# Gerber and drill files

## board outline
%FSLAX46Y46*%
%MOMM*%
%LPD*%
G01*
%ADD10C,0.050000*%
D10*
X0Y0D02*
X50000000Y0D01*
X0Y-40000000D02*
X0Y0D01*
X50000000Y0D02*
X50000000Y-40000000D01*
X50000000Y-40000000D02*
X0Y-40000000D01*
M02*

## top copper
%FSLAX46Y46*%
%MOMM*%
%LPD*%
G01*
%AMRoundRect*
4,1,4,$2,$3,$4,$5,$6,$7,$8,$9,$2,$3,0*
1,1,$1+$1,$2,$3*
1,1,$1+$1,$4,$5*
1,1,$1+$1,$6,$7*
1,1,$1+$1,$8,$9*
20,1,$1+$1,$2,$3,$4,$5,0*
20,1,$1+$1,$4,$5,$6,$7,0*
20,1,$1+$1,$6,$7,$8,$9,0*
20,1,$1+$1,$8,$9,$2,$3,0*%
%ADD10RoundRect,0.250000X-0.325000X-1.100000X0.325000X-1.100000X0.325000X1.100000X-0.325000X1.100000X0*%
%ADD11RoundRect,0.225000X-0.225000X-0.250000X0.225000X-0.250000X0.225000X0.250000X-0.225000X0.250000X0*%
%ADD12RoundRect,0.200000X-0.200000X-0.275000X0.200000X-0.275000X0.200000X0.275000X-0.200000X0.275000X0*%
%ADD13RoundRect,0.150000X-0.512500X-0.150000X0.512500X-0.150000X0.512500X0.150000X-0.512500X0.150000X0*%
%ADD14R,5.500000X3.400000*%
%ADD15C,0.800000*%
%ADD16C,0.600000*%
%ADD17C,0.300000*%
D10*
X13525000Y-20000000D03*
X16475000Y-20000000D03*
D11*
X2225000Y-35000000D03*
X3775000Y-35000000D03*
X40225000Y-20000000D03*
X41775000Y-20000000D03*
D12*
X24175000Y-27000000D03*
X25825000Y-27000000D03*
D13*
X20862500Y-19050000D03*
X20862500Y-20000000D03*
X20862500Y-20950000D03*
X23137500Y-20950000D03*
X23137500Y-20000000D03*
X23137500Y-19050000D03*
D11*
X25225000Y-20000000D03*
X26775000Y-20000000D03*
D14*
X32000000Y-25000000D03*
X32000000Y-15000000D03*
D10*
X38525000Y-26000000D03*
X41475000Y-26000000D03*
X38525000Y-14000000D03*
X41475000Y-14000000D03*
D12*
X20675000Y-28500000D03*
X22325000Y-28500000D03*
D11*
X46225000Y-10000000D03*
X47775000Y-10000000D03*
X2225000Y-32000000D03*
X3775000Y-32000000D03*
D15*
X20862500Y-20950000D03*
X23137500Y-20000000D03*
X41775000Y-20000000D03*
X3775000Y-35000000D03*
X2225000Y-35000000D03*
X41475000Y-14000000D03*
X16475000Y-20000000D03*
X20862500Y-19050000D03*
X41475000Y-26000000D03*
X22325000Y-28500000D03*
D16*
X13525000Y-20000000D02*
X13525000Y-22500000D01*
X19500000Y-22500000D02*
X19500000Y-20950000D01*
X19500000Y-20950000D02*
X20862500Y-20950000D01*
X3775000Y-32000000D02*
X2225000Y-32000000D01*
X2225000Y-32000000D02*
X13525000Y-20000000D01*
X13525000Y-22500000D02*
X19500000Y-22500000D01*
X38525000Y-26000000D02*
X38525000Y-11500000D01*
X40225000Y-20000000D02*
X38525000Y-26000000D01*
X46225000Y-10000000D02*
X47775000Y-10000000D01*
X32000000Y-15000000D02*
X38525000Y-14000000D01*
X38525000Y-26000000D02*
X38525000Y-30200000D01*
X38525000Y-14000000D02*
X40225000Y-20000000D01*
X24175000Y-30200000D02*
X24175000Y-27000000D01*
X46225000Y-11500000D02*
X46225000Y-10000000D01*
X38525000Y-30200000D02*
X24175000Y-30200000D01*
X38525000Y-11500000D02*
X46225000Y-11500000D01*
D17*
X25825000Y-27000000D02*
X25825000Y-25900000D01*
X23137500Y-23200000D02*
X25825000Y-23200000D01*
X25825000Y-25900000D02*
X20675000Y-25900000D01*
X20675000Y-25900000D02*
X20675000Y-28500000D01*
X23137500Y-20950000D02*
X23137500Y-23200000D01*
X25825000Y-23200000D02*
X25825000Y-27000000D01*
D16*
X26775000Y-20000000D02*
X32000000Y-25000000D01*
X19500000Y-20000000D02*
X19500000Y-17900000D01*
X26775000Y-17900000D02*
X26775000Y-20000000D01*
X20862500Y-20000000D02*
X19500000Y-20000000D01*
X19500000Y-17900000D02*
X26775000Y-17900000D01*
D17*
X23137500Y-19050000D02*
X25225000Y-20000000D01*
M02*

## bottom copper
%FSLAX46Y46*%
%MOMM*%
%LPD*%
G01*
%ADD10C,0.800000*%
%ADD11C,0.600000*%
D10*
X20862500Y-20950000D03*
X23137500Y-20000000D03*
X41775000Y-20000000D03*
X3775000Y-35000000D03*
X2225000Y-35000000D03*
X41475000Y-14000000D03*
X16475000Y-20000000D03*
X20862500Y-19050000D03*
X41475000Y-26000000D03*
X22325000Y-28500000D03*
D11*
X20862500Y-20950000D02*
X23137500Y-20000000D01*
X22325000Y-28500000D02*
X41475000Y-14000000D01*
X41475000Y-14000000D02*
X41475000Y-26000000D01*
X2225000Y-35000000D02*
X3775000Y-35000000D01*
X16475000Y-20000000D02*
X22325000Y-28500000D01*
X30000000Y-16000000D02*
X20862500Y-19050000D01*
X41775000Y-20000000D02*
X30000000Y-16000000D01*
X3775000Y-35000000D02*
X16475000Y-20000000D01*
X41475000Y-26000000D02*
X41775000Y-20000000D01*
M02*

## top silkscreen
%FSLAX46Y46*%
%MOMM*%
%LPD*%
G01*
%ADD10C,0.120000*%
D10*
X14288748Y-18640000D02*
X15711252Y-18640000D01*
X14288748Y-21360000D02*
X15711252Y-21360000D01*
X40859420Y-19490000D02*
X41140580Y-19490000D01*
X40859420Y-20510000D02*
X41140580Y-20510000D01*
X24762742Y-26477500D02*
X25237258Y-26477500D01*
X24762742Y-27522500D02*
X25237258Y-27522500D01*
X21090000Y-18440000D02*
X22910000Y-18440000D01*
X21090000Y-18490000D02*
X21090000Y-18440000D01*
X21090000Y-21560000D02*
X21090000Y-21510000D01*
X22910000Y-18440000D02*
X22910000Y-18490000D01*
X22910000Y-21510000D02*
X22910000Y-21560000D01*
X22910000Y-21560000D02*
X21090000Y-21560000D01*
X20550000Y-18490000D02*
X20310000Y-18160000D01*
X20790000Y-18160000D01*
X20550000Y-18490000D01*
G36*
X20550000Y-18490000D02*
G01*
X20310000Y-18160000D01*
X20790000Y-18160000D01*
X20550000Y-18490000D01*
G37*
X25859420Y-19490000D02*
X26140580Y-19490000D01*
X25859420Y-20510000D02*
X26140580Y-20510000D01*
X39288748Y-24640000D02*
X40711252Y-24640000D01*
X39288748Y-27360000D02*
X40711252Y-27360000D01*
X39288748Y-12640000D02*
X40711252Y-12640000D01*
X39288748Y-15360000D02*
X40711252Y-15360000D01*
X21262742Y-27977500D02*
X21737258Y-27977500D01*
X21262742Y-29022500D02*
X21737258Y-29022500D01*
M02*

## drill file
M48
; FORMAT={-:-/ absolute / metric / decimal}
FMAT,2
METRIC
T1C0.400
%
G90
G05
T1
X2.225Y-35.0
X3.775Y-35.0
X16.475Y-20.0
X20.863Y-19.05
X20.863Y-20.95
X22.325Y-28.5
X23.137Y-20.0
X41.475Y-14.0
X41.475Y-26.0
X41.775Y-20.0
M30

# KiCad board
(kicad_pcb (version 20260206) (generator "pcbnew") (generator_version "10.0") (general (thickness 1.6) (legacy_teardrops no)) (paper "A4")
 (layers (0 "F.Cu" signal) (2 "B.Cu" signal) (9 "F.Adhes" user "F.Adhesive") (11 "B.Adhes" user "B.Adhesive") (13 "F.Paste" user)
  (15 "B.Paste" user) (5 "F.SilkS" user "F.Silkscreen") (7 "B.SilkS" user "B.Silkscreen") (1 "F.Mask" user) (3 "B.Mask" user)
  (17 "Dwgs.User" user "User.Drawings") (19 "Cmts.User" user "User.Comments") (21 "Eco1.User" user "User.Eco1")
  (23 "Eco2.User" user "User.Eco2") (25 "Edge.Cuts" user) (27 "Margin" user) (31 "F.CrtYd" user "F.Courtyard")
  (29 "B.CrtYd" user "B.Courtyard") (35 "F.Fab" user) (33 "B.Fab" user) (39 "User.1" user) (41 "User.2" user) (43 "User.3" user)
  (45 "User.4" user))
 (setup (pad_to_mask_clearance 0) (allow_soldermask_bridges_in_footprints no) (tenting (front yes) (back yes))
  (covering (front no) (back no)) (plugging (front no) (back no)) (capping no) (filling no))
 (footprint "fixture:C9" (layer "F.Cu") (at 15 20)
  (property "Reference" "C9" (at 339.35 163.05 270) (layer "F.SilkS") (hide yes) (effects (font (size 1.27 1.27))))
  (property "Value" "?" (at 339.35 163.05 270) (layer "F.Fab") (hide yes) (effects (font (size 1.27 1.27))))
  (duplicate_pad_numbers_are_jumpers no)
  (fp_line (start -0.711252 -1.36) (end 0.711252 -1.36) (stroke (width 0.12) (type solid)) (layer "F.SilkS"))
  (fp_line (start -0.711252 1.36) (end 0.711252 1.36) (stroke (width 0.12) (type solid)) (layer "F.SilkS"))
  (pad "1" smd roundrect (at -1.475 0) (size 1.15 2.7) (layers "F.Cu" "F.Mask" "F.Paste") (roundrect_rratio 0.217391) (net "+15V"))
  (pad "2" smd roundrect (at 1.475 0) (size 1.15 2.7) (layers "F.Cu" "F.Mask" "F.Paste") (roundrect_rratio 0.217391) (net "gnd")))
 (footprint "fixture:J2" (layer "F.Cu") (at 3 35)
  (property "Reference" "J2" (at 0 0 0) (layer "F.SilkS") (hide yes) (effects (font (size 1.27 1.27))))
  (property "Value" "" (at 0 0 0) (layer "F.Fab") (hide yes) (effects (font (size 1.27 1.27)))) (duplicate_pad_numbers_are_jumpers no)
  (pad "1" smd roundrect (at -0.775 0) (size 0.9 0.95) (layers "F.Cu" "F.Mask" "F.Paste") (roundrect_rratio 0.25) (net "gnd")
   (thermal_bridge_angle 45))
  (pad "2" smd roundrect (at 0.775 0) (size 0.9 0.95) (layers "F.Cu" "F.Mask" "F.Paste") (roundrect_rratio 0.25) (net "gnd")
   (thermal_bridge_angle 45)))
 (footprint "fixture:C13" (layer "F.Cu") (at 41 20)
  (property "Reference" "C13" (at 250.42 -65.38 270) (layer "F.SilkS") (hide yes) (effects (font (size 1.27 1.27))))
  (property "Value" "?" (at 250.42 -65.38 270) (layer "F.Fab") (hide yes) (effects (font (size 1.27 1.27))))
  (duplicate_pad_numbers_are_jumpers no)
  (fp_line (start -0.14058 -0.51) (end 0.14058 -0.51) (stroke (width 0.12) (type solid)) (layer "F.SilkS"))
  (fp_line (start -0.14058 0.51) (end 0.14058 0.51) (stroke (width 0.12) (type solid)) (layer "F.SilkS"))
  (pad "1" smd roundrect (at -0.775 0) (size 0.9 0.95) (layers "F.Cu" "F.Mask" "F.Paste") (roundrect_rratio 0.25) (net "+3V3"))
  (pad "2" smd roundrect (at 0.775 0) (size 0.9 0.95) (layers "F.Cu" "F.Mask" "F.Paste") (roundrect_rratio 0.25) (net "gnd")))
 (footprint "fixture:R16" (layer "F.Cu") (at 25 27)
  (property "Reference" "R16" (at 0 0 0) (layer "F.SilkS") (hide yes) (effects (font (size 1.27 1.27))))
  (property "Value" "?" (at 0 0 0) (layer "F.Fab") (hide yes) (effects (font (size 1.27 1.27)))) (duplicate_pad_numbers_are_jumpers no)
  (fp_line (start -0.237258 -0.5225) (end 0.237258 -0.5225) (stroke (width 0.12) (type solid)) (layer "F.SilkS"))
  (fp_line (start -0.237258 0.5225) (end 0.237258 0.5225) (stroke (width 0.12) (type solid)) (layer "F.SilkS"))
  (pad "1" smd roundrect (at -0.825 0) (size 0.8 0.95) (layers "F.Cu" "F.Mask" "F.Paste") (roundrect_rratio 0.25) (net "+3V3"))
  (pad "2" smd roundrect (at 0.825 0) (size 0.8 0.95) (layers "F.Cu" "F.Mask" "F.Paste") (roundrect_rratio 0.25) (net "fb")))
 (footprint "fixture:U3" (layer "F.Cu") (at 22 20)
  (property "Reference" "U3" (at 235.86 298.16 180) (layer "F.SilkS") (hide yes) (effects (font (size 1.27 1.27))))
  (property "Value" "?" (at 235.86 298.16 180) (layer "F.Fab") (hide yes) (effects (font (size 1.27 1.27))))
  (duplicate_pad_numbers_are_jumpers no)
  (fp_line (start -0.91 -1.56) (end 0.91 -1.56) (stroke (width 0.12) (type solid)) (layer "F.SilkS"))
  (fp_line (start -0.91 -1.51) (end -0.91 -1.56) (stroke (width 0.12) (type solid)) (layer "F.SilkS"))
  (fp_line (start -0.91 1.56) (end -0.91 1.51) (stroke (width 0.12) (type solid)) (layer "F.SilkS"))
  (fp_line (start 0.91 -1.56) (end 0.91 -1.51) (stroke (width 0.12) (type solid)) (layer "F.SilkS"))
  (fp_line (start 0.91 1.51) (end 0.91 1.56) (stroke (width 0.12) (type solid)) (layer "F.SilkS"))
  (fp_line (start 0.91 1.56) (end -0.91 1.56) (stroke (width 0.12) (type solid)) (layer "F.SilkS"))
  (fp_poly (pts (xy -1.45 -1.51) (xy -1.69 -1.84) (xy -1.21 -1.84)) (stroke (width 0.12) (type solid)) (fill yes) (layer "F.SilkS"))
  (pad "1" smd roundrect (at -1.1375 -0.95) (size 1.325 0.6) (layers "F.Cu" "F.Mask" "F.Paste") (roundrect_rratio 0.25) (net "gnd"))
  (pad "2" smd roundrect (at -1.1375 0) (size 1.325 0.6) (layers "F.Cu" "F.Mask" "F.Paste") (roundrect_rratio 0.25) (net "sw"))
  (pad "3" smd roundrect (at -1.1375 0.95) (size 1.325 0.6) (layers "F.Cu" "F.Mask" "F.Paste") (roundrect_rratio 0.25) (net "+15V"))
  (pad "4" smd roundrect (at 1.1375 0.95) (size 1.325 0.6) (layers "F.Cu" "F.Mask" "F.Paste") (roundrect_rratio 0.25) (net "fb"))
  (pad "5" smd roundrect (at 1.1375 0) (size 1.325 0.6) (layers "F.Cu" "F.Mask" "F.Paste") (roundrect_rratio 0.25) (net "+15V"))
  (pad "6" smd roundrect (at 1.1375 -0.95) (size 1.325 0.6) (layers "F.Cu" "F.Mask" "F.Paste") (roundrect_rratio 0.25) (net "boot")))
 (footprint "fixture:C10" (layer "F.Cu") (at 26 20)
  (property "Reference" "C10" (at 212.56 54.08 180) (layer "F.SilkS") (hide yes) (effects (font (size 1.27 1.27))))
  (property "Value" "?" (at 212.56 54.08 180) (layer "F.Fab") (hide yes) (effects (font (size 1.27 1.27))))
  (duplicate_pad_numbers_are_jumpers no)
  (fp_line (start -0.14058 -0.51) (end 0.14058 -0.51) (stroke (width 0.12) (type solid)) (layer "F.SilkS"))
  (fp_line (start -0.14058 0.51) (end 0.14058 0.51) (stroke (width 0.12) (type solid)) (layer "F.SilkS"))
  (pad "1" smd roundrect (at -0.775 0) (size 0.9 0.95) (layers "F.Cu" "F.Mask" "F.Paste") (roundrect_rratio 0.25) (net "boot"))
  (pad "2" smd roundrect (at 0.775 0) (size 0.9 0.95) (layers "F.Cu" "F.Mask" "F.Paste") (roundrect_rratio 0.25) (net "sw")))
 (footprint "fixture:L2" (layer "F.Cu") (at 32 20 90)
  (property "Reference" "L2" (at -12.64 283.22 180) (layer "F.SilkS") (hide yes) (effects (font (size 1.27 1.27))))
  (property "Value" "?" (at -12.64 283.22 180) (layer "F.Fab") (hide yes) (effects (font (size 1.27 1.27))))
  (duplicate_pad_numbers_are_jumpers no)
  (pad "1" smd rect (at -5 0 90) (size 3.4 5.5) (layers "F.Cu" "F.Mask" "F.Paste") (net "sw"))
  (pad "2" smd rect (at 5 0 90) (size 3.4 5.5) (layers "F.Cu" "F.Mask" "F.Paste") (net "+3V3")))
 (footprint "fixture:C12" (layer "F.Cu") (at 40 26)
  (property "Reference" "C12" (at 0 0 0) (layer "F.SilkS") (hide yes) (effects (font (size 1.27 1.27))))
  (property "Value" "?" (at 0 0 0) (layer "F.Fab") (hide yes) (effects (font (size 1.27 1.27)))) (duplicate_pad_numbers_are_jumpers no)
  (fp_line (start -0.711252 -1.36) (end 0.711252 -1.36) (stroke (width 0.12) (type solid)) (layer "F.SilkS"))
  (fp_line (start -0.711252 1.36) (end 0.711252 1.36) (stroke (width 0.12) (type solid)) (layer "F.SilkS"))
  (pad "1" smd roundrect (at -1.475 0) (size 1.15 2.7) (layers "F.Cu" "F.Mask" "F.Paste") (roundrect_rratio 0.217391) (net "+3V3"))
  (pad "2" smd roundrect (at 1.475 0) (size 1.15 2.7) (layers "F.Cu" "F.Mask" "F.Paste") (roundrect_rratio 0.217391) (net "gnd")))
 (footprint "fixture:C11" (layer "F.Cu") (at 40 14)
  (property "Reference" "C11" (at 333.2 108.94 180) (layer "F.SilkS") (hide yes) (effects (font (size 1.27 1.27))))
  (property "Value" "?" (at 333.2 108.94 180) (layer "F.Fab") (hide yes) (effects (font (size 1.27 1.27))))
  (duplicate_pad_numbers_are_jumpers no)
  (fp_line (start -0.711252 -1.36) (end 0.711252 -1.36) (stroke (width 0.12) (type solid)) (layer "F.SilkS"))
  (fp_line (start -0.711252 1.36) (end 0.711252 1.36) (stroke (width 0.12) (type solid)) (layer "F.SilkS"))
  (pad "1" smd roundrect (at -1.475 0) (size 1.15 2.7) (layers "F.Cu" "F.Mask" "F.Paste") (roundrect_rratio 0.217391) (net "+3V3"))
  (pad "2" smd roundrect (at 1.475 0) (size 1.15 2.7) (layers "F.Cu" "F.Mask" "F.Paste") (roundrect_rratio 0.217391) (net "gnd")))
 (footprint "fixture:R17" (layer "F.Cu") (at 21.5 28.5)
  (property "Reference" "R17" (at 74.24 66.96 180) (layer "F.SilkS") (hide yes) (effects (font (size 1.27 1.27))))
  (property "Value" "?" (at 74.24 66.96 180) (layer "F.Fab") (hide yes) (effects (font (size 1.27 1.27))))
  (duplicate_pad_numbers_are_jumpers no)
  (fp_line (start -0.237258 -0.5225) (end 0.237258 -0.5225) (stroke (width 0.12) (type solid)) (layer "F.SilkS"))
  (fp_line (start -0.237258 0.5225) (end 0.237258 0.5225) (stroke (width 0.12) (type solid)) (layer "F.SilkS"))
  (pad "1" smd roundrect (at -0.825 0) (size 0.8 0.95) (layers "F.Cu" "F.Mask" "F.Paste") (roundrect_rratio 0.25) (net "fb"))
  (pad "2" smd roundrect (at 0.825 0) (size 0.8 0.95) (layers "F.Cu" "F.Mask" "F.Paste") (roundrect_rratio 0.25) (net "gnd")))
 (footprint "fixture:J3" (layer "F.Cu") (at 47 10)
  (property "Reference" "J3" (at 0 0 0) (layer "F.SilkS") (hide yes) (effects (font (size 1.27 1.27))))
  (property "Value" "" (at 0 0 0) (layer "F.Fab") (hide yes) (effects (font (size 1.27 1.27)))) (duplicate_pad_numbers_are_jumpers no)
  (pad "1" smd roundrect (at -0.775 0) (size 0.9 0.95) (layers "F.Cu" "F.Mask" "F.Paste") (roundrect_rratio 0.25) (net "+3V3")
   (thermal_bridge_angle 45))
  (pad "2" smd roundrect (at 0.775 0) (size 0.9 0.95) (layers "F.Cu" "F.Mask" "F.Paste") (roundrect_rratio 0.25) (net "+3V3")
   (thermal_bridge_angle 45)))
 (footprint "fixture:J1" (layer "F.Cu") (at 3 32)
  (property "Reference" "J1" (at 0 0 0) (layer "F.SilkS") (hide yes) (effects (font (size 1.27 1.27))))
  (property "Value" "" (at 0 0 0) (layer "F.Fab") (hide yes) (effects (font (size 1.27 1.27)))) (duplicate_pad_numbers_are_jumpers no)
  (pad "1" smd roundrect (at -0.775 0) (size 0.9 0.95) (layers "F.Cu" "F.Mask" "F.Paste") (roundrect_rratio 0.25) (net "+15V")
   (thermal_bridge_angle 45))
  (pad "2" smd roundrect (at 0.775 0) (size 0.9 0.95) (layers "F.Cu" "F.Mask" "F.Paste") (roundrect_rratio 0.25) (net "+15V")
   (thermal_bridge_angle 45)))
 (gr_line (start 0 0) (end 50 0) (stroke (width 0.05) (type default)) (layer "Edge.Cuts"))
 (gr_line (start 0 40) (end 0 0) (stroke (width 0.05) (type default)) (layer "Edge.Cuts"))
 (gr_line (start 50 0) (end 50 40) (stroke (width 0.05) (type default)) (layer "Edge.Cuts"))
 (gr_line (start 50 40) (end 0 40) (stroke (width 0.05) (type default)) (layer "Edge.Cuts"))
 (segment (start 13.525 20) (end 13.525 22.5) (width 0.6) (layer "F.Cu") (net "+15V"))
 (segment (start 19.5 22.5) (end 19.5 20.95) (width 0.6) (layer "F.Cu") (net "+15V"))
 (segment (start 19.5 20.95) (end 20.8625 20.95) (width 0.6) (layer "F.Cu") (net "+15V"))
 (segment (start 3.775 32) (end 2.225 32) (width 0.6) (layer "F.Cu") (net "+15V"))
 (segment (start 2.225 32) (end 13.525 20) (width 0.6) (layer "F.Cu") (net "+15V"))
 (segment (start 13.525 22.5) (end 19.5 22.5) (width 0.6) (layer "F.Cu") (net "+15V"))
 (via (at 20.8625 20.95) (size 0.8) (drill 0.4) (layers "F.Cu" "B.Cu") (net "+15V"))
 (via (at 23.1375 20) (size 0.8) (drill 0.4) (layers "F.Cu" "B.Cu") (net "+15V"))
 (segment (start 20.8625 20.95) (end 23.1375 20) (width 0.6) (layer "B.Cu") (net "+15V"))
 (via (at 41.775 20) (size 0.8) (drill 0.4) (layers "F.Cu" "B.Cu") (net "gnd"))
 (via (at 3.775 35) (size 0.8) (drill 0.4) (layers "F.Cu" "B.Cu") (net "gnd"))
 (via (at 2.225 35) (size 0.8) (drill 0.4) (layers "F.Cu" "B.Cu") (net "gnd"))
 (via (at 41.475 14) (size 0.8) (drill 0.4) (layers "F.Cu" "B.Cu") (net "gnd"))
 (via (at 16.475 20) (size 0.8) (drill 0.4) (layers "F.Cu" "B.Cu") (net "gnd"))
 (via (at 20.8625 19.05) (size 0.8) (drill 0.4) (layers "F.Cu" "B.Cu") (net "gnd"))
 (via (at 41.475 26) (size 0.8) (drill 0.4) (layers "F.Cu" "B.Cu") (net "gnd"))
 (via (at 22.325 28.5) (size 0.8) (drill 0.4) (layers "F.Cu" "B.Cu") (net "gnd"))
 (segment (start 22.325 28.5) (end 41.475 14) (width 0.6) (layer "B.Cu") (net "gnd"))
 (segment (start 41.475 14) (end 41.475 26) (width 0.6) (layer "B.Cu") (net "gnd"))
 (segment (start 2.225 35) (end 3.775 35) (width 0.6) (layer "B.Cu") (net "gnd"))
 (segment (start 16.475 20) (end 22.325 28.5) (width 0.6) (layer "B.Cu") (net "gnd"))
 (segment (start 30 16) (end 20.8625 19.05) (width 0.6) (layer "B.Cu") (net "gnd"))
 (segment (start 41.775 20) (end 30 16) (width 0.6) (layer "B.Cu") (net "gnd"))
 (segment (start 3.775 35) (end 16.475 20) (width 0.6) (layer "B.Cu") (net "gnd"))
 (segment (start 41.475 26) (end 41.775 20) (width 0.6) (layer "B.Cu") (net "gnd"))
 (segment (start 38.525 26) (end 38.525 11.5) (width 0.6) (layer "F.Cu") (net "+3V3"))
 (segment (start 40.225 20) (end 38.525 26) (width 0.6) (layer "F.Cu") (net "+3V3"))
 (segment (start 46.225 10) (end 47.775 10) (width 0.6) (layer "F.Cu") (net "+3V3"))
 (segment (start 32 15) (end 38.525 14) (width 0.6) (layer "F.Cu") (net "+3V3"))
 (segment (start 38.525 26) (end 38.525 30.2) (width 0.6) (layer "F.Cu") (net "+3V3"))
 (segment (start 38.525 14) (end 40.225 20) (width 0.6) (layer "F.Cu") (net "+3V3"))
 (segment (start 24.175 30.2) (end 24.175 27) (width 0.6) (layer "F.Cu") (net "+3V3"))
 (segment (start 46.225 11.5) (end 46.225 10) (width 0.6) (layer "F.Cu") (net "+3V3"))
 (segment (start 38.525 30.2) (end 24.175 30.2) (width 0.6) (layer "F.Cu") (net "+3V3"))
 (segment (start 38.525 11.5) (end 46.225 11.5) (width 0.6) (layer "F.Cu") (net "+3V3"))
 (segment (start 25.825 27) (end 25.825 25.9) (width 0.3) (layer "F.Cu") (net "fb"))
 (segment (start 23.1375 23.2) (end 25.825 23.2) (width 0.3) (layer "F.Cu") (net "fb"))
 (segment (start 25.825 25.9) (end 20.675 25.9) (width 0.3) (layer "F.Cu") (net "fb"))
 (segment (start 20.675 25.9) (end 20.675 28.5) (width 0.3) (layer "F.Cu") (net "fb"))
 (segment (start 23.1375 20.95) (end 23.1375 23.2) (width 0.3) (layer "F.Cu") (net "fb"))
 (segment (start 25.825 23.2) (end 25.825 27) (width 0.3) (layer "F.Cu") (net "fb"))
 (segment (start 26.775 20) (end 32 25) (width 0.6) (layer "F.Cu") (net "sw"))
 (segment (start 19.5 20) (end 19.5 17.9) (width 0.6) (layer "F.Cu") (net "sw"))
 (segment (start 26.775 17.9) (end 26.775 20) (width 0.6) (layer "F.Cu") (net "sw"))
 (segment (start 20.8625 20) (end 19.5 20) (width 0.6) (layer "F.Cu") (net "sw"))
 (segment (start 19.5 17.9) (end 26.775 17.9) (width 0.6) (layer "F.Cu") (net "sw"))
 (segment (start 23.1375 19.05) (end 25.225 20) (width 0.3) (layer "F.Cu") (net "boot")))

